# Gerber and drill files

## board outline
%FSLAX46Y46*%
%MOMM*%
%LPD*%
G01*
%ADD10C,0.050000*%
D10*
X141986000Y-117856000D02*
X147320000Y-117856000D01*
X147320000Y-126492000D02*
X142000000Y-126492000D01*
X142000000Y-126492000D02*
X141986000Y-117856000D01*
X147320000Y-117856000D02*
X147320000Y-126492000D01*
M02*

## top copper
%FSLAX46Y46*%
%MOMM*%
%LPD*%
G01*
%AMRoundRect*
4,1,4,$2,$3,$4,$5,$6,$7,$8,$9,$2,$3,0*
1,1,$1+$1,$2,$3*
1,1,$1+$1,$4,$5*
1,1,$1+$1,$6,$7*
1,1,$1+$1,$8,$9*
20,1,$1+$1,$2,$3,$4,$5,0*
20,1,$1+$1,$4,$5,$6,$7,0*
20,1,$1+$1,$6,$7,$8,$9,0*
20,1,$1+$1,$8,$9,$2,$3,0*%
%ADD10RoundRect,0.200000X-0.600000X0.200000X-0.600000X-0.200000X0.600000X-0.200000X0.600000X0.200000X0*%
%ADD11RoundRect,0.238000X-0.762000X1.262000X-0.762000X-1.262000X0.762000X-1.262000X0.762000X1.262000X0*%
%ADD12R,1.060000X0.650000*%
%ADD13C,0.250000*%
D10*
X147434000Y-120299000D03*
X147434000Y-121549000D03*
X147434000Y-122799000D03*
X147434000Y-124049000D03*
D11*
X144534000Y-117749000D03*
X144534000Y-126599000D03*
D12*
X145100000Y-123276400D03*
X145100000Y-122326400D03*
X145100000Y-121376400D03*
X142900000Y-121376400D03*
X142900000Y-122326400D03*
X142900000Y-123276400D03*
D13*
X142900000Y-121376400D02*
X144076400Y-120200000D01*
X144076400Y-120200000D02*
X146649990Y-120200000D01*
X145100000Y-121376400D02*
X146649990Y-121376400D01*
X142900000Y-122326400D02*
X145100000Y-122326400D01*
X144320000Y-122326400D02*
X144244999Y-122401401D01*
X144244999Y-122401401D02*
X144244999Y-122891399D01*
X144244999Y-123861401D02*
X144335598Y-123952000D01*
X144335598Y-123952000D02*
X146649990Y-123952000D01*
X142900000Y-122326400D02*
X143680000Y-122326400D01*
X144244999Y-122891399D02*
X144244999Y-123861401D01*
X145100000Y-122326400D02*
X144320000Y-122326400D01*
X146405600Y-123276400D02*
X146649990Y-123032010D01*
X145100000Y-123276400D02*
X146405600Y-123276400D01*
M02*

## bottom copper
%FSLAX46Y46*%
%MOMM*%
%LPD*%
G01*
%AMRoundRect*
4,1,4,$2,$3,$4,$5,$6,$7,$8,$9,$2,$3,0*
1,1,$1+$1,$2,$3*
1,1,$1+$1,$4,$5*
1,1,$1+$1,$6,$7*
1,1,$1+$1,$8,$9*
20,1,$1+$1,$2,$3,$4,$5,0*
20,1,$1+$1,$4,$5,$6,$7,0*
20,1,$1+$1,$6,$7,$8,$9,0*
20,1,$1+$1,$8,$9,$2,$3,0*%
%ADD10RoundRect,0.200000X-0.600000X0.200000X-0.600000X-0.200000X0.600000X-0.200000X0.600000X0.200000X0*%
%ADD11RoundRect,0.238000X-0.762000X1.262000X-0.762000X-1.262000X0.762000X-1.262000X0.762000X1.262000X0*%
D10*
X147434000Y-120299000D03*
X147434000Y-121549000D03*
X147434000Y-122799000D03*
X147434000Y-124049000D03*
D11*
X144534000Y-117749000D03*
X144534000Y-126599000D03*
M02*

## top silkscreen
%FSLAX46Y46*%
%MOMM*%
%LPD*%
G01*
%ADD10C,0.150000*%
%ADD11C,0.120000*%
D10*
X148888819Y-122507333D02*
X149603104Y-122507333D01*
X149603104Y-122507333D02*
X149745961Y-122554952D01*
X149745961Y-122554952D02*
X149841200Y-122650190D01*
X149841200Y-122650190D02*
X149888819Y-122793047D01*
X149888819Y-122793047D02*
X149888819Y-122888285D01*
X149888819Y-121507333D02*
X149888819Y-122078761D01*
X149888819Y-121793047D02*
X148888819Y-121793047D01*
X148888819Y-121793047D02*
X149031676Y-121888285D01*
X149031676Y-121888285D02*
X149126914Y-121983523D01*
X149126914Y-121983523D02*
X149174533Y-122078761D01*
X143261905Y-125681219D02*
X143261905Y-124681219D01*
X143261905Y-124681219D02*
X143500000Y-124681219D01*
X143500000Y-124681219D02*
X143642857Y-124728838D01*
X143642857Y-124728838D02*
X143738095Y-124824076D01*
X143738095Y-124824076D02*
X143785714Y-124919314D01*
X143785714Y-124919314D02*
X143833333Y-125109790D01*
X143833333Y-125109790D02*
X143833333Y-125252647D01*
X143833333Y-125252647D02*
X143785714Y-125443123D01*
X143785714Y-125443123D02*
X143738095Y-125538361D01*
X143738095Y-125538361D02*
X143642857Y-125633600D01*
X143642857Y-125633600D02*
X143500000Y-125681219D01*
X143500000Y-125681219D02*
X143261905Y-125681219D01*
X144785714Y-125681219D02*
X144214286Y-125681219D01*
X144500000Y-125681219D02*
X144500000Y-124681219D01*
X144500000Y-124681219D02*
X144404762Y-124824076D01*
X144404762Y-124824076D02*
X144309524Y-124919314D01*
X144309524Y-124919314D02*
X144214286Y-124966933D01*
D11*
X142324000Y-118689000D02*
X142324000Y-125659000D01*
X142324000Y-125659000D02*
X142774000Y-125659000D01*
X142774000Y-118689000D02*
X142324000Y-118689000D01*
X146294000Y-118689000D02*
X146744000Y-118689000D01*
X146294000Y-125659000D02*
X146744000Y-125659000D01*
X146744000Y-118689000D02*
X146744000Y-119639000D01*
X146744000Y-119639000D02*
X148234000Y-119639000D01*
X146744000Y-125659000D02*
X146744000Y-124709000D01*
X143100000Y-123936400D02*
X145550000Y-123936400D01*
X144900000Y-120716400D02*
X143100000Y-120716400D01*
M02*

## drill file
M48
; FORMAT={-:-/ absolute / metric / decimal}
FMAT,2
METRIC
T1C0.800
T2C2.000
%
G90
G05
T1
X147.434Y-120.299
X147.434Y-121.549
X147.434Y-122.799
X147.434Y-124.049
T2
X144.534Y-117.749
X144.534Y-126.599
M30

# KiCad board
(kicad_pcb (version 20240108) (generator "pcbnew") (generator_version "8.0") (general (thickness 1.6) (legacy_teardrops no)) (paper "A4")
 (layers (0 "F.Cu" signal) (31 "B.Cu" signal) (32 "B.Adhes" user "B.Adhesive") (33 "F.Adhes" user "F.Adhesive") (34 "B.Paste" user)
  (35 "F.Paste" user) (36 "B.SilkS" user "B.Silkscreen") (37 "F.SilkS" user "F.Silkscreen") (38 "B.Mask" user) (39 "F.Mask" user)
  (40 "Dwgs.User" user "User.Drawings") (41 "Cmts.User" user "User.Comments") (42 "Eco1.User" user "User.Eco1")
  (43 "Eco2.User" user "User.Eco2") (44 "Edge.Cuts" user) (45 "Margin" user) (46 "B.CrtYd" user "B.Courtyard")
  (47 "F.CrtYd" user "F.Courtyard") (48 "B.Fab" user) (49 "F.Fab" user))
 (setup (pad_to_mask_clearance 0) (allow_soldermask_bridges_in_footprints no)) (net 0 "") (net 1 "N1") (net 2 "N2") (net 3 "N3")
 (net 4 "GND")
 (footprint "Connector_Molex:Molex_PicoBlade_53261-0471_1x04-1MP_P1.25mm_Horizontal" (layer "F.Cu") (at 145.034 122.174 -90)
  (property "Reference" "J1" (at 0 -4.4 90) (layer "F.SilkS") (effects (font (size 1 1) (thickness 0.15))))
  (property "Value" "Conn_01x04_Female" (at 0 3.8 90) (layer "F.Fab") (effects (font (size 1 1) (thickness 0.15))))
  (fp_line (start -3.485 2.71) (end 3.485 2.71) (stroke (width 0.12) (type solid)) (layer "F.SilkS"))
  (fp_line (start 3.485 2.71) (end 3.485 2.26) (stroke (width 0.12) (type solid)) (layer "F.SilkS"))
  (fp_line (start -3.485 2.26) (end -3.485 2.71) (stroke (width 0.12) (type solid)) (layer "F.SilkS"))
  (fp_line (start -3.485 -1.26) (end -3.485 -1.71) (stroke (width 0.12) (type solid)) (layer "F.SilkS"))
  (fp_line (start 3.485 -1.26) (end 3.485 -1.71) (stroke (width 0.12) (type solid)) (layer "F.SilkS"))
  (fp_line (start -3.485 -1.71) (end -2.535 -1.71) (stroke (width 0.12) (type solid)) (layer "F.SilkS"))
  (fp_line (start -2.535 -1.71) (end -2.535 -3.2) (stroke (width 0.12) (type solid)) (layer "F.SilkS"))
  (fp_line (start 3.485 -1.71) (end 2.535 -1.71) (stroke (width 0.12) (type solid)) (layer "F.SilkS"))
  (pad "1" thru_hole roundrect (at -1.875 -2.4 270) (size 0.8 1.6) (drill 0.8) (layers "*.Cu" "*.Mask") (remove_unused_layers no)
   (roundrect_rratio 0.25) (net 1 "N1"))
  (pad "2" thru_hole roundrect (at -0.625 -2.4 270) (size 0.8 1.6) (drill 0.8) (layers "*.Cu" "*.Mask") (remove_unused_layers no)
   (roundrect_rratio 0.25) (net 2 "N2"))
  (pad "3" thru_hole roundrect (at 0.625 -2.4 270) (size 0.8 1.6) (drill 0.8) (layers "*.Cu" "*.Mask") (remove_unused_layers no)
   (roundrect_rratio 0.25) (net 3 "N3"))
  (pad "4" thru_hole roundrect (at 1.875 -2.4 270) (size 0.8 1.6) (drill 0.8) (layers "*.Cu" "*.Mask") (remove_unused_layers no)
   (roundrect_rratio 0.25) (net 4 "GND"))
  (pad "MP" thru_hole roundrect (at -4.425 0.5 270) (size 3 2) (drill 2) (layers "*.Cu" "*.Mask") (remove_unused_layers no)
   (roundrect_rratio 0.119))
  (pad "MP" thru_hole roundrect (at 4.425 0.5 270) (size 3 2) (drill 2) (layers "*.Cu" "*.Mask") (remove_unused_layers no)
   (roundrect_rratio 0.119)))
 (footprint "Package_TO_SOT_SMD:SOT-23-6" (layer "F.Cu") (at 144 122.3264 180)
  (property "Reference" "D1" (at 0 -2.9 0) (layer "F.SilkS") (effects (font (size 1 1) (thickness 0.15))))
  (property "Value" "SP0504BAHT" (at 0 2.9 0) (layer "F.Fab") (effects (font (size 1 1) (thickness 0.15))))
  (fp_line (start 0.9 -1.61) (end -1.55 -1.61) (stroke (width 0.12) (type solid)) (layer "F.SilkS"))
  (fp_line (start -0.9 1.61) (end 0.9 1.61) (stroke (width 0.12) (type solid)) (layer "F.SilkS"))
  (pad "1" smd rect (at -1.1 -0.95 180) (size 1.06 0.65) (layers "F.Cu" "F.Paste" "F.Mask") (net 3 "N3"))
  (pad "2" smd rect (at -1.1 0 180) (size 1.06 0.65) (layers "F.Cu" "F.Paste" "F.Mask") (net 4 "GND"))
  (pad "3" smd rect (at -1.1 0.95 180) (size 1.06 0.65) (layers "F.Cu" "F.Paste" "F.Mask") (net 2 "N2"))
  (pad "4" smd rect (at 1.1 0.95 180) (size 1.06 0.65) (layers "F.Cu" "F.Paste" "F.Mask") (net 1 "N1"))
  (pad "5" smd rect (at 1.1 0 180) (size 1.06 0.65) (layers "F.Cu" "F.Paste" "F.Mask") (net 4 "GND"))
  (pad "6" smd rect (at 1.1 -0.95 180) (size 1.06 0.65) (layers "F.Cu" "F.Paste" "F.Mask")))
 (gr_line (start 141.986 117.856) (end 147.32 117.856) (stroke (width 0.05) (type solid)) (layer "Edge.Cuts"))
 (gr_line (start 147.32 126.492) (end 142 126.492) (stroke (width 0.05) (type solid)) (layer "Edge.Cuts"))
 (gr_line (start 142 126.492) (end 141.986 117.856) (stroke (width 0.05) (type solid)) (layer "Edge.Cuts"))
 (gr_line (start 147.32 117.856) (end 147.32 126.492) (stroke (width 0.05) (type solid)) (layer "Edge.Cuts"))
 (segment (start 142.9 121.3764) (end 144.0764 120.2) (width 0.25) (layer "F.Cu") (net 1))
 (segment (start 144.0764 120.2) (end 146.64999 120.2) (width 0.25) (layer "F.Cu") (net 1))
 (segment (start 145.1 121.3764) (end 146.64999 121.3764) (width 0.25) (layer "F.Cu") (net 2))
 (segment (start 142.9 122.3264) (end 145.1 122.3264) (width 0.25) (layer "F.Cu") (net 4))
 (segment (start 144.32 122.3264) (end 144.244999 122.401401) (width 0.25) (layer "F.Cu") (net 4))
 (segment (start 144.244999 122.401401) (end 144.244999 122.891399) (width 0.25) (layer "F.Cu") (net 4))
 (segment (start 144.244999 123.861401) (end 144.335598 123.952) (width 0.25) (layer "F.Cu") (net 4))
 (segment (start 144.335598 123.952) (end 146.64999 123.952) (width 0.25) (layer "F.Cu") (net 4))
 (segment (start 142.9 122.3264) (end 143.68 122.3264) (width 0.25) (layer "F.Cu") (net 4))
 (segment (start 144.244999 122.891399) (end 144.244999 123.861401) (width 0.25) (layer "F.Cu") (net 4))
 (segment (start 145.1 122.3264) (end 144.32 122.3264) (width 0.25) (layer "F.Cu") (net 4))
 (segment (start 146.4056 123.2764) (end 146.64999 123.03201) (width 0.25) (layer "F.Cu") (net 3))
 (segment (start 145.1 123.2764) (end 146.4056 123.2764) (width 0.25) (layer "F.Cu") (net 3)))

